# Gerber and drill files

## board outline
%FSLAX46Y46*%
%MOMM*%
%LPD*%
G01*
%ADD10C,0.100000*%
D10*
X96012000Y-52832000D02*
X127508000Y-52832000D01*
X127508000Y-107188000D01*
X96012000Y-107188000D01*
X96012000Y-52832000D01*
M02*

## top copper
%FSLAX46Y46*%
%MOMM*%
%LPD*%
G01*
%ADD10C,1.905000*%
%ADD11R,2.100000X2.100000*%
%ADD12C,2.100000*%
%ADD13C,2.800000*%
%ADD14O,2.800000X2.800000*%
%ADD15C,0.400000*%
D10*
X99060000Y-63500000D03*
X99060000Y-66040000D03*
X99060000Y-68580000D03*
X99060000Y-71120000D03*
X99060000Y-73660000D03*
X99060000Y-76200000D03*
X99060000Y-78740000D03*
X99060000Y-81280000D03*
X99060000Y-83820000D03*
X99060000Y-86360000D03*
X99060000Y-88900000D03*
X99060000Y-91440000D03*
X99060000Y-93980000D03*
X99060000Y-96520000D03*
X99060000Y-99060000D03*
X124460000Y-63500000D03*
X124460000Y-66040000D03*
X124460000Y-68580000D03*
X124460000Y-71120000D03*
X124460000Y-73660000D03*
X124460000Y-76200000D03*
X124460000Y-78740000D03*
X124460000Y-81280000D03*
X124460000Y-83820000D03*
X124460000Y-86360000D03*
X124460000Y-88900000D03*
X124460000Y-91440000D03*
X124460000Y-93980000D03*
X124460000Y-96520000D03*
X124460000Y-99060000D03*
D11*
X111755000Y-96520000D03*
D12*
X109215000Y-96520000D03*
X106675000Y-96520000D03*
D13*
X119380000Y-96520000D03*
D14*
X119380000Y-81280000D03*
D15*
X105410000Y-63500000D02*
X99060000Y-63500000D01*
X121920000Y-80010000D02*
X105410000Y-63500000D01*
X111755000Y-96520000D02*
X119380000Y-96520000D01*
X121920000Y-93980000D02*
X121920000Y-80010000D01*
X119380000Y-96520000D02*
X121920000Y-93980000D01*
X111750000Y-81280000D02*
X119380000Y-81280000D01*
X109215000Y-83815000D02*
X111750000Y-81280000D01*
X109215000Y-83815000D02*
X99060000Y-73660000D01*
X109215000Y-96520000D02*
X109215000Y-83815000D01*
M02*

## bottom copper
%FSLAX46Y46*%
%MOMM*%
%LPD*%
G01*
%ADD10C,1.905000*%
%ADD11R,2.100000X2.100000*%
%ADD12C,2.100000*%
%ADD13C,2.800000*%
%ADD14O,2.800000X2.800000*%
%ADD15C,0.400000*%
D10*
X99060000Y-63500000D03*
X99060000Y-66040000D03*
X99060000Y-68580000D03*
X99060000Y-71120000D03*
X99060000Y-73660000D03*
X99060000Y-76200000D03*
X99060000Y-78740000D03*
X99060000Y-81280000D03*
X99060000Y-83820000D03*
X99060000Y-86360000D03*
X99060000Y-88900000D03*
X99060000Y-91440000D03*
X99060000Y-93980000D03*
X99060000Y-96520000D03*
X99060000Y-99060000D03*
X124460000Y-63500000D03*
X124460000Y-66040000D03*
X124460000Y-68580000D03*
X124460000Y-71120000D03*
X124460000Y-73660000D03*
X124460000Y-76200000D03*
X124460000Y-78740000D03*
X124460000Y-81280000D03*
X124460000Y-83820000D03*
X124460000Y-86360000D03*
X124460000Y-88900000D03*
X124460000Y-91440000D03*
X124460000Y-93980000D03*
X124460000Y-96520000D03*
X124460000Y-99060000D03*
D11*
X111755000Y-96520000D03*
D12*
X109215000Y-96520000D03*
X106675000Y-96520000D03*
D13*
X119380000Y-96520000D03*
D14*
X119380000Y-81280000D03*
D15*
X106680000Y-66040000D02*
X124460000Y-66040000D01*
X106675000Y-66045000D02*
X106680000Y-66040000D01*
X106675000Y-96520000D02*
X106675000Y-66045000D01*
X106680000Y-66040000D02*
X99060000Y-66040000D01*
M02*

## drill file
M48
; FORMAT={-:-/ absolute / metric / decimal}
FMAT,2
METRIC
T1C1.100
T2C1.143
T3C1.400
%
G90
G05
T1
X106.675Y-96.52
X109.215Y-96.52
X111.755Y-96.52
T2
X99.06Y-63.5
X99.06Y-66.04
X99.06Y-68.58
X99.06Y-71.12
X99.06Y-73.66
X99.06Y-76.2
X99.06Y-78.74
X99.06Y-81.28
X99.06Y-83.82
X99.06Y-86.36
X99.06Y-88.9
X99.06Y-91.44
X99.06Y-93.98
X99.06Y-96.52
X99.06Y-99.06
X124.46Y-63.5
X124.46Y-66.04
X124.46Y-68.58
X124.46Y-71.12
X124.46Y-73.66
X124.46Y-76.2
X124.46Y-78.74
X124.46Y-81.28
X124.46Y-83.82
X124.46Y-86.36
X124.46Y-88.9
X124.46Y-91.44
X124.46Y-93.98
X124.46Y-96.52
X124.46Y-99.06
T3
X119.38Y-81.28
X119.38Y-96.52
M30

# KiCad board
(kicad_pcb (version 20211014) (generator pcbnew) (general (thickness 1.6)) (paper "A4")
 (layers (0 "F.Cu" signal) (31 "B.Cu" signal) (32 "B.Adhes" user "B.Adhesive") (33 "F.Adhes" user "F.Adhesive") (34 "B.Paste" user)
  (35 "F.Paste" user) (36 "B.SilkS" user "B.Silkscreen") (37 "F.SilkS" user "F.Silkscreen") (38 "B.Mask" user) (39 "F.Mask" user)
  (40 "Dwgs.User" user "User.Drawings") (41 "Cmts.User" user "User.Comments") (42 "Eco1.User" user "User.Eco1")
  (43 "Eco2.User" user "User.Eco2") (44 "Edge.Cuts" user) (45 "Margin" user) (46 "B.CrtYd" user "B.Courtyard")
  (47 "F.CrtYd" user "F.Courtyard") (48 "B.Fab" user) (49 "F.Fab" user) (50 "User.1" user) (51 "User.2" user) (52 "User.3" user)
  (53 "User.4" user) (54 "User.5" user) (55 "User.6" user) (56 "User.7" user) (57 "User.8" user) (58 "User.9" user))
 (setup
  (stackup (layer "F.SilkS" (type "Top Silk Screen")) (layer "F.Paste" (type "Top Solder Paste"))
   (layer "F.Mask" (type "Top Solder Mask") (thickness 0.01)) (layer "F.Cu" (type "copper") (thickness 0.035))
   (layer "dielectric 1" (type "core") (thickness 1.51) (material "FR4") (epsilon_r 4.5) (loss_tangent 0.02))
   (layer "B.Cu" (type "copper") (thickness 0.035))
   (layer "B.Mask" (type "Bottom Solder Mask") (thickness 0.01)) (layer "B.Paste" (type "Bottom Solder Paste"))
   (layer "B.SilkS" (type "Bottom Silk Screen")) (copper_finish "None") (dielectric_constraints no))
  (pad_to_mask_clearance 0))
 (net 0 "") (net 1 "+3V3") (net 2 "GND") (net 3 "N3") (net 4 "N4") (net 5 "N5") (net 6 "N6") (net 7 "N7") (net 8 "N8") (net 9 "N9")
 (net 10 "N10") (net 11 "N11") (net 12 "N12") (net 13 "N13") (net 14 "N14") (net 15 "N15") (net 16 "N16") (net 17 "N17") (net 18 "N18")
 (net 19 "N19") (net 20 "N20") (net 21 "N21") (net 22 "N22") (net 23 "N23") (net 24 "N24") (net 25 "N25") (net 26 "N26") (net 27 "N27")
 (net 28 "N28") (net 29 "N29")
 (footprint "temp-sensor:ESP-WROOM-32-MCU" (layer "F.Cu") (at 111.76 80.01)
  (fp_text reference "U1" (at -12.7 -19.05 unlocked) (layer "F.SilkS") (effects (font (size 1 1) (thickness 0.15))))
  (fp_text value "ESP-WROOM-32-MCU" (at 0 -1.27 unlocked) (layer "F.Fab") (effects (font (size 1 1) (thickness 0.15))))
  (pad "1" thru_hole circle (at -12.7 -16.51) (size 1.905 1.905) (drill 1.143) (layers *.Cu *.Mask) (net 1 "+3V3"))
  (pad "2" thru_hole circle (at -12.7 -13.97) (size 1.905 1.905) (drill 1.143) (layers *.Cu *.Mask) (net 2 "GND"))
  (pad "3" thru_hole circle (at -12.7 -11.43) (size 1.905 1.905) (drill 1.143) (layers *.Cu *.Mask) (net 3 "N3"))
  (pad "4" thru_hole circle (at -12.7 -8.89) (size 1.905 1.905) (drill 1.143) (layers *.Cu *.Mask) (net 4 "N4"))
  (pad "5" thru_hole circle (at -12.7 -6.35) (size 1.905 1.905) (drill 1.143) (layers *.Cu *.Mask) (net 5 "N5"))
  (pad "6" thru_hole circle (at -12.7 -3.81) (size 1.905 1.905) (drill 1.143) (layers *.Cu *.Mask) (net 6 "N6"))
  (pad "7" thru_hole circle (at -12.7 -1.27) (size 1.905 1.905) (drill 1.143) (layers *.Cu *.Mask) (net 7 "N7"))
  (pad "8" thru_hole circle (at -12.7 1.27) (size 1.905 1.905) (drill 1.143) (layers *.Cu *.Mask) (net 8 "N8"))
  (pad "9" thru_hole circle (at -12.7 3.81) (size 1.905 1.905) (drill 1.143) (layers *.Cu *.Mask) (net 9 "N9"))
  (pad "10" thru_hole circle (at -12.7 6.35) (size 1.905 1.905) (drill 1.143) (layers *.Cu *.Mask) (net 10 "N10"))
  (pad "11" thru_hole circle (at -12.7 8.89) (size 1.905 1.905) (drill 1.143) (layers *.Cu *.Mask) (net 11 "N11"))
  (pad "12" thru_hole circle (at -12.7 11.43) (size 1.905 1.905) (drill 1.143) (layers *.Cu *.Mask) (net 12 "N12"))
  (pad "13" thru_hole circle (at -12.7 13.97) (size 1.905 1.905) (drill 1.143) (layers *.Cu *.Mask) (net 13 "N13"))
  (pad "14" thru_hole circle (at -12.7 16.51) (size 1.905 1.905) (drill 1.143) (layers *.Cu *.Mask) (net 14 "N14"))
  (pad "15" thru_hole circle (at -12.7 19.05) (size 1.905 1.905) (drill 1.143) (layers *.Cu *.Mask) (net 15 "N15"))
  (pad "16" thru_hole circle (at 12.7 -16.51) (size 1.905 1.905) (drill 1.143) (layers *.Cu *.Mask) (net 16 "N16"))
  (pad "17" thru_hole circle (at 12.7 -13.97) (size 1.905 1.905) (drill 1.143) (layers *.Cu *.Mask) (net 2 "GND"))
  (pad "18" thru_hole circle (at 12.7 -11.43) (size 1.905 1.905) (drill 1.143) (layers *.Cu *.Mask) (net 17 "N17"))
  (pad "19" thru_hole circle (at 12.7 -8.89) (size 1.905 1.905) (drill 1.143) (layers *.Cu *.Mask) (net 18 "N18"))
  (pad "20" thru_hole circle (at 12.7 -6.35) (size 1.905 1.905) (drill 1.143) (layers *.Cu *.Mask) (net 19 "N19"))
  (pad "21" thru_hole circle (at 12.7 -3.81) (size 1.905 1.905) (drill 1.143) (layers *.Cu *.Mask) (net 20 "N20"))
  (pad "22" thru_hole circle (at 12.7 -1.27) (size 1.905 1.905) (drill 1.143) (layers *.Cu *.Mask) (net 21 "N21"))
  (pad "23" thru_hole circle (at 12.7 1.27) (size 1.905 1.905) (drill 1.143) (layers *.Cu *.Mask) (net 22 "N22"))
  (pad "24" thru_hole circle (at 12.7 3.81) (size 1.905 1.905) (drill 1.143) (layers *.Cu *.Mask) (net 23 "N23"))
  (pad "25" thru_hole circle (at 12.7 6.35) (size 1.905 1.905) (drill 1.143) (layers *.Cu *.Mask) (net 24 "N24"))
  (pad "26" thru_hole circle (at 12.7 8.89) (size 1.905 1.905) (drill 1.143) (layers *.Cu *.Mask) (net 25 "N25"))
  (pad "27" thru_hole circle (at 12.7 11.43) (size 1.905 1.905) (drill 1.143) (layers *.Cu *.Mask) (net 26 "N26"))
  (pad "28" thru_hole circle (at 12.7 13.97) (size 1.905 1.905) (drill 1.143) (layers *.Cu *.Mask) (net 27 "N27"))
  (pad "29" thru_hole circle (at 12.7 16.51) (size 1.905 1.905) (drill 1.143) (layers *.Cu *.Mask) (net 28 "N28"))
  (pad "30" thru_hole circle (at 12.7 19.05) (size 1.905 1.905) (drill 1.143) (layers *.Cu *.Mask) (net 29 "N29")))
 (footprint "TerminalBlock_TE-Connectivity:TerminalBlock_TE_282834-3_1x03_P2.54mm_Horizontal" (layer "B.Cu") (at 111.755 96.52 180)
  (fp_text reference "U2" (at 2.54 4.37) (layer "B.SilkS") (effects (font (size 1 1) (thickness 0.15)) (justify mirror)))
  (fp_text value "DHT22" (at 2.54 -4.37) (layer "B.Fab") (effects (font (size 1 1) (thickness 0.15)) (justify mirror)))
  (pad "1" thru_hole rect (at 0 0 180) (size 2.1 2.1) (drill 1.1) (layers *.Cu *.Mask) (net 1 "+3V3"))
  (pad "2" thru_hole circle (at 2.54 0 180) (size 2.1 2.1) (drill 1.1) (layers *.Cu *.Mask) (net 5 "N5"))
  (pad "3" thru_hole circle (at 5.08 0 180) (size 2.1 2.1) (drill 1.1) (layers *.Cu *.Mask) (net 2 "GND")))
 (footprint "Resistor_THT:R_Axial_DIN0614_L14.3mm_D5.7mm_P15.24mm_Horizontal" (layer "B.Cu") (at 119.38 96.52 90)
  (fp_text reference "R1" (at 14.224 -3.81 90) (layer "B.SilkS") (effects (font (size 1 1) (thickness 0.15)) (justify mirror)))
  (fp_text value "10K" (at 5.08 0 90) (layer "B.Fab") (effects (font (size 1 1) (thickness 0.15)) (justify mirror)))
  (pad "1" thru_hole circle (at 0 0 90) (size 2.8 2.8) (drill 1.4) (layers *.Cu *.Mask) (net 1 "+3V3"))
  (pad "2" thru_hole oval (at 15.24 0 90) (size 2.8 2.8) (drill 1.4) (layers *.Cu *.Mask) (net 5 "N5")))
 (gr_rect (start 96.012 52.832) (end 127.508 107.188) (layer "Edge.Cuts") (width 0.1) (fill none))
 (segment (start 105.41 63.5) (end 99.06 63.5) (width 0.4) (layer "F.Cu") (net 1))
 (segment (start 121.92 80.01) (end 105.41 63.5) (width 0.4) (layer "F.Cu") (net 1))
 (segment (start 111.755 96.52) (end 119.38 96.52) (width 0.4) (layer "F.Cu") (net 1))
 (segment (start 121.92 93.98) (end 121.92 80.01) (width 0.4) (layer "F.Cu") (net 1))
 (segment (start 119.38 96.52) (end 121.92 93.98) (width 0.4) (layer "F.Cu") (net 1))
 (segment (start 106.68 66.04) (end 124.46 66.04) (width 0.4) (layer "B.Cu") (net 2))
 (segment (start 106.675 66.045) (end 106.68 66.04) (width 0.4) (layer "B.Cu") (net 2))
 (segment (start 106.675 96.52) (end 106.675 66.045) (width 0.4) (layer "B.Cu") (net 2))
 (segment (start 106.68 66.04) (end 99.06 66.04) (width 0.4) (layer "B.Cu") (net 2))
 (segment (start 111.75 81.28) (end 119.38 81.28) (width 0.4) (layer "F.Cu") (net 5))
 (segment (start 109.215 83.815) (end 111.75 81.28) (width 0.4) (layer "F.Cu") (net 5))
 (segment (start 109.215 83.815) (end 99.06 73.66) (width 0.4) (layer "F.Cu") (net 5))
 (segment (start 109.215 96.52) (end 109.215 83.815) (width 0.4) (layer "F.Cu") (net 5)))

